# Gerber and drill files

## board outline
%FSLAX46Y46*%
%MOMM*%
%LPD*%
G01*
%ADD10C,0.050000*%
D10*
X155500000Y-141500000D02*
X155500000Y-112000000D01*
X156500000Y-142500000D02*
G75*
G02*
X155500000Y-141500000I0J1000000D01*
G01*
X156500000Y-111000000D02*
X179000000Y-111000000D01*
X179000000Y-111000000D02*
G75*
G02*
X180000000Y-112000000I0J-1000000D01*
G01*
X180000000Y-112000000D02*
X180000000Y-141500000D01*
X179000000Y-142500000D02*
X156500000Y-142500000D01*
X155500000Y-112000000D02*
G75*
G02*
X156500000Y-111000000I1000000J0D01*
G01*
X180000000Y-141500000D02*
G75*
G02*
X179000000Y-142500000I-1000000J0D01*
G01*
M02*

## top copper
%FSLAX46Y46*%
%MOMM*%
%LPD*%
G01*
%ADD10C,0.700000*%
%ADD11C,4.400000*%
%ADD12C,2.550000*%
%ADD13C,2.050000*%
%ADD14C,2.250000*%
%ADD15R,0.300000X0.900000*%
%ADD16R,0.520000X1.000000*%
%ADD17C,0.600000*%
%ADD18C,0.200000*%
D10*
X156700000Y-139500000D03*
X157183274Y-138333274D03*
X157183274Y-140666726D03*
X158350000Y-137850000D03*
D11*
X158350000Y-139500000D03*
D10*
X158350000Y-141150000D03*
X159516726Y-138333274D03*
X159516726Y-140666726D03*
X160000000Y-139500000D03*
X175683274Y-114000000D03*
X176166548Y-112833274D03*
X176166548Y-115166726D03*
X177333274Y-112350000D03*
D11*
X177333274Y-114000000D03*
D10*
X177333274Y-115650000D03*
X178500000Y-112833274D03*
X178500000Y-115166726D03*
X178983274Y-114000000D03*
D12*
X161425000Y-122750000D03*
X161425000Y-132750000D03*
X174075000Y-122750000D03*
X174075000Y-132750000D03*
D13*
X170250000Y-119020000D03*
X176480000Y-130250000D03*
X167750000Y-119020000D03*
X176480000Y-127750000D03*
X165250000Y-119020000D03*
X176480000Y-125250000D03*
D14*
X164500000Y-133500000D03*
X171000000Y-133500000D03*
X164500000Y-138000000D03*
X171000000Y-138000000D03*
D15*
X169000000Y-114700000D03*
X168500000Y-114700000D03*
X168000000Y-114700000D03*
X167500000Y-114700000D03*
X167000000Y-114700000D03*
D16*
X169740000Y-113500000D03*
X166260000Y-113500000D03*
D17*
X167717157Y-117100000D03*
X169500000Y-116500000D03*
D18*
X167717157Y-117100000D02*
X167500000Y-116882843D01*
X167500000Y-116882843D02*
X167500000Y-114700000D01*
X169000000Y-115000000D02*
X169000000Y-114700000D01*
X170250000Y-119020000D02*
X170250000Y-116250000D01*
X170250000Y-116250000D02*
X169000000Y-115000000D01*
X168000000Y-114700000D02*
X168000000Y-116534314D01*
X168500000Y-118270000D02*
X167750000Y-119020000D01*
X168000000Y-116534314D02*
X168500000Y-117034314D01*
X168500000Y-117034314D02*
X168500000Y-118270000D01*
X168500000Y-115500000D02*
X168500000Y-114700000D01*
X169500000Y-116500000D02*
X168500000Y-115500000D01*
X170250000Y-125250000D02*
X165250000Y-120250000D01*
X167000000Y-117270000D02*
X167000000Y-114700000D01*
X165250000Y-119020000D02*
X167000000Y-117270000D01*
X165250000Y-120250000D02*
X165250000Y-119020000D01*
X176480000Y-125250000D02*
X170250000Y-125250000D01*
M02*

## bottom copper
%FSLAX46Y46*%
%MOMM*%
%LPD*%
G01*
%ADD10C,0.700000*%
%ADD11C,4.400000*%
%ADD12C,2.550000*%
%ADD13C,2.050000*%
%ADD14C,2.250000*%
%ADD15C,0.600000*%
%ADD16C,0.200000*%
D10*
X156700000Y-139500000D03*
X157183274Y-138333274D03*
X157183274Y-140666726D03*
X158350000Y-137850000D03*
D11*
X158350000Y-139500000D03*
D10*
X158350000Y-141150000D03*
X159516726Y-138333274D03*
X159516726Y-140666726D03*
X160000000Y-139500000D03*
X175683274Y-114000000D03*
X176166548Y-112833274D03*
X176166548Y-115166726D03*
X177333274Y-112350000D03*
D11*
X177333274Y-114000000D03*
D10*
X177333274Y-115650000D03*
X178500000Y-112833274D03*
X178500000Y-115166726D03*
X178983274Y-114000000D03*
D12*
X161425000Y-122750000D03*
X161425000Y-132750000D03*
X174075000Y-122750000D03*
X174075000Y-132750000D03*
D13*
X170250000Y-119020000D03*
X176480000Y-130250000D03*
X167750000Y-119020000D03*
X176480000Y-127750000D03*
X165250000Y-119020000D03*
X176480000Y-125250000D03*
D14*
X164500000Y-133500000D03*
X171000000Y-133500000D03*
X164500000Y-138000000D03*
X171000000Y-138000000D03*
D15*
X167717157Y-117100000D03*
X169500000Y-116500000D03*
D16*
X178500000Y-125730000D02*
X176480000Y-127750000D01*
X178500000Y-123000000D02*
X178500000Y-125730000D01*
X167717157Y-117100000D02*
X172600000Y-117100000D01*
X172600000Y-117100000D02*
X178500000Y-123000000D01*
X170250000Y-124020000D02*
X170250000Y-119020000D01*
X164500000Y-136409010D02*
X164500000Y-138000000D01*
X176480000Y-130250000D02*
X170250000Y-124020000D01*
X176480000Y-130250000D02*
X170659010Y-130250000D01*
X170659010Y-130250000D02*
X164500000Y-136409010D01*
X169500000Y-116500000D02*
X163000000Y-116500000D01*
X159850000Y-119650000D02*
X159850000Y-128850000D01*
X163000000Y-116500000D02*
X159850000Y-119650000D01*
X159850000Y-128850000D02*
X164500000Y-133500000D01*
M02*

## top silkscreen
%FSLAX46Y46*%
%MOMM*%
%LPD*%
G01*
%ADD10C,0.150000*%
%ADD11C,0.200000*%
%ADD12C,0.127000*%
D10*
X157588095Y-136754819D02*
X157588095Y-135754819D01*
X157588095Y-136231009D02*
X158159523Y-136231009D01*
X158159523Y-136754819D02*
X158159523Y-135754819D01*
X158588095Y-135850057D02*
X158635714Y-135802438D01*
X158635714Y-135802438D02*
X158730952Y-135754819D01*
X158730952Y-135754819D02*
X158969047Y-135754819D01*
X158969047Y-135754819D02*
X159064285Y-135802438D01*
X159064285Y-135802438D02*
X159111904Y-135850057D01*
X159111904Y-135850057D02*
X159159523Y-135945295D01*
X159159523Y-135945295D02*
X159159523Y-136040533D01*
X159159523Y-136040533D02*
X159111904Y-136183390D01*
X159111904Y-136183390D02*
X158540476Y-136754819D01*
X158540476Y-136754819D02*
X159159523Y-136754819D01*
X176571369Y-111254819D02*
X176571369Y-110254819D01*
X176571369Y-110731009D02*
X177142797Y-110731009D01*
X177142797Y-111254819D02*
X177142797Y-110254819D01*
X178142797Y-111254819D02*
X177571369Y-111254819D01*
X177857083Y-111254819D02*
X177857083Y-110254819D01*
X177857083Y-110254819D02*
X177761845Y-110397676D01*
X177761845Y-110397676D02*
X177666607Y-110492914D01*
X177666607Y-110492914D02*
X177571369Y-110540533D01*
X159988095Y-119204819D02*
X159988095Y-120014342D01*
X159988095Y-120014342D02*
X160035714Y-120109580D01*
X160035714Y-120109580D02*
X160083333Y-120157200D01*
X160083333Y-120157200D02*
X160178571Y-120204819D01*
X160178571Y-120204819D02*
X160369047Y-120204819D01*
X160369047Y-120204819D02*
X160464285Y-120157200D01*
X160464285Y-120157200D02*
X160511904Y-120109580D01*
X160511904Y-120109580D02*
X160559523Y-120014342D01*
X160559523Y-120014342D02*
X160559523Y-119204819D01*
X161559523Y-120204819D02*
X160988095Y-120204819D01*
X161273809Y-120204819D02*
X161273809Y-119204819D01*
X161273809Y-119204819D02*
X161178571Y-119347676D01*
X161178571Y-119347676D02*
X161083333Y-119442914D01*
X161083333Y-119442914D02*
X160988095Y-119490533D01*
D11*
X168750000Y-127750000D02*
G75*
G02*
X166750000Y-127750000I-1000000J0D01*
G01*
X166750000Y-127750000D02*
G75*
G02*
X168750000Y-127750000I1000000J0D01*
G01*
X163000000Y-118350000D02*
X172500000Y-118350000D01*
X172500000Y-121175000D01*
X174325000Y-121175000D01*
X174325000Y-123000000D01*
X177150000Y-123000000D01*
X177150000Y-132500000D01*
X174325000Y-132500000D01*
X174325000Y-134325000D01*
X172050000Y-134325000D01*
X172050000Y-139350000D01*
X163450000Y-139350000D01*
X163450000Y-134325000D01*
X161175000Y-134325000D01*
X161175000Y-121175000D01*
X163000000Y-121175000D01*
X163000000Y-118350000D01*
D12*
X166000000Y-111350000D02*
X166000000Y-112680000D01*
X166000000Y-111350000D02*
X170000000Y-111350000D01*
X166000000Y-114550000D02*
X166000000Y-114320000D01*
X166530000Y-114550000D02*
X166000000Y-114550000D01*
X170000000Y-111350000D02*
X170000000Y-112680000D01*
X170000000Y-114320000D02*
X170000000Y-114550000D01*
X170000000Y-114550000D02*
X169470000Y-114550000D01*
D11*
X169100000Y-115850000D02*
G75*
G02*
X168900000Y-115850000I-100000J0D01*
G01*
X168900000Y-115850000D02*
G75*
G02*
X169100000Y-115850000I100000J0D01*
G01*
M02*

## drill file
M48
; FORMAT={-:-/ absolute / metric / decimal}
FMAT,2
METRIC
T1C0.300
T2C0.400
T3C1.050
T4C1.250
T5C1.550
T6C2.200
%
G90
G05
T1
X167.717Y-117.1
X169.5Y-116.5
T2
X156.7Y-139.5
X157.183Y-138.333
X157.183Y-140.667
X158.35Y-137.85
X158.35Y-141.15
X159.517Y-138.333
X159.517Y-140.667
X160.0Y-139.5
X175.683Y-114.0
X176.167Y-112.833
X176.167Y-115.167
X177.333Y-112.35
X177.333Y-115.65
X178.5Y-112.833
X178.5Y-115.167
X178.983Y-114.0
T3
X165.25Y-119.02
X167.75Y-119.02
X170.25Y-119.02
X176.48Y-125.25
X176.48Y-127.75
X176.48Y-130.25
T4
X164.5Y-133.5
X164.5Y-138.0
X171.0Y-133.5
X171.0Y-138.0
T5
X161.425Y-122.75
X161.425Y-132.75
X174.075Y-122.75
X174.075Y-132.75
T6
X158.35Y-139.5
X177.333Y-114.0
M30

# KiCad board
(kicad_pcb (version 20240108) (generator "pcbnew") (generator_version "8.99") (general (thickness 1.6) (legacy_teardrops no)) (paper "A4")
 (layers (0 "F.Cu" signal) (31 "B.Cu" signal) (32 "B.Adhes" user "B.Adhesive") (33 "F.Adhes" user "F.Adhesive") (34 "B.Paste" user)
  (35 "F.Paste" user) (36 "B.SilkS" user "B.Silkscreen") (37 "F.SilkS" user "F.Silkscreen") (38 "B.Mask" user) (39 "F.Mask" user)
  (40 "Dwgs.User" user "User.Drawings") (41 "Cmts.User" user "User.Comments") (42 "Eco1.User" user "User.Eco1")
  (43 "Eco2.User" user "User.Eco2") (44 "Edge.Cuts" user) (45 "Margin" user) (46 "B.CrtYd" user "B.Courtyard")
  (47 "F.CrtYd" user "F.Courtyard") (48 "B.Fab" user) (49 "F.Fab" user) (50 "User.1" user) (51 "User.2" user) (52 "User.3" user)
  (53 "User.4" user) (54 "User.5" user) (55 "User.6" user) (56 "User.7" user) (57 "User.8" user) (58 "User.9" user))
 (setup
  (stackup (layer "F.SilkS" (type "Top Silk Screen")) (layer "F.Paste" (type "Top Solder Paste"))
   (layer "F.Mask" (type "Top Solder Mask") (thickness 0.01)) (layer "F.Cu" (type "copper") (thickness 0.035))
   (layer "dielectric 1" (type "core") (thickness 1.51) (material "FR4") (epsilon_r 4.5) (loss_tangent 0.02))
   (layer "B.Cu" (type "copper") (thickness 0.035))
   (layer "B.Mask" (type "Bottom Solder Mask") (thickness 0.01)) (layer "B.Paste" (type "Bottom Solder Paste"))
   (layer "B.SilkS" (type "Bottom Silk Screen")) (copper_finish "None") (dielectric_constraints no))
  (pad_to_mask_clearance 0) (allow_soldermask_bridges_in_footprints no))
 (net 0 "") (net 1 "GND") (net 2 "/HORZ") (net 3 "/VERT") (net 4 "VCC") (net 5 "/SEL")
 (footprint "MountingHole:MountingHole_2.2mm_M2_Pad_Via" (layer "F.Cu") (at 158.35 139.5)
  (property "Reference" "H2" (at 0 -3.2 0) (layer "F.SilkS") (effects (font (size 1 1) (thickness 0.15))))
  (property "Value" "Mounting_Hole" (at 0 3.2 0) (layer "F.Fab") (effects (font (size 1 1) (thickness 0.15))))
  (pad "1" thru_hole circle (at -1.65 0) (size 0.7 0.7) (drill 0.4) (layers "*.Cu" "*.Mask") (remove_unused_layers no) (zone_connect 2))
  (pad "1" thru_hole circle (at -1.166726 -1.166726) (size 0.7 0.7) (drill 0.4) (layers "*.Cu" "*.Mask") (remove_unused_layers no)
   (zone_connect 2))
  (pad "1" thru_hole circle (at -1.166726 1.166726) (size 0.7 0.7) (drill 0.4) (layers "*.Cu" "*.Mask") (remove_unused_layers no)
   (zone_connect 2))
  (pad "1" thru_hole circle (at 0 -1.65) (size 0.7 0.7) (drill 0.4) (layers "*.Cu" "*.Mask") (remove_unused_layers no) (zone_connect 2))
  (pad "1" thru_hole circle (at 0 0) (size 4.4 4.4) (drill 2.2) (layers "*.Cu" "*.Mask") (remove_unused_layers no))
  (pad "1" thru_hole circle (at 0 1.65) (size 0.7 0.7) (drill 0.4) (layers "*.Cu" "*.Mask") (remove_unused_layers no) (zone_connect 2))
  (pad "1" thru_hole circle (at 1.166726 -1.166726) (size 0.7 0.7) (drill 0.4) (layers "*.Cu" "*.Mask") (remove_unused_layers no)
   (zone_connect 2))
  (pad "1" thru_hole circle (at 1.166726 1.166726) (size 0.7 0.7) (drill 0.4) (layers "*.Cu" "*.Mask") (remove_unused_layers no)
   (zone_connect 2))
  (pad "1" thru_hole circle (at 1.65 0) (size 0.7 0.7) (drill 0.4) (layers "*.Cu" "*.Mask") (remove_unused_layers no) (zone_connect 2)))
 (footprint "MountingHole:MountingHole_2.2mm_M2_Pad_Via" (layer "F.Cu") (at 177.333274 114)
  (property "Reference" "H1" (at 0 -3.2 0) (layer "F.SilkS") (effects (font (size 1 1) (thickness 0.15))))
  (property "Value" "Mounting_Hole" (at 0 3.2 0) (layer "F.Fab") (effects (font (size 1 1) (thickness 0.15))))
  (pad "1" thru_hole circle (at -1.65 0) (size 0.7 0.7) (drill 0.4) (layers "*.Cu" "*.Mask") (remove_unused_layers no) (zone_connect 2))
  (pad "1" thru_hole circle (at -1.166726 -1.166726) (size 0.7 0.7) (drill 0.4) (layers "*.Cu" "*.Mask") (remove_unused_layers no)
   (zone_connect 2))
  (pad "1" thru_hole circle (at -1.166726 1.166726) (size 0.7 0.7) (drill 0.4) (layers "*.Cu" "*.Mask") (remove_unused_layers no)
   (zone_connect 2))
  (pad "1" thru_hole circle (at 0 -1.65) (size 0.7 0.7) (drill 0.4) (layers "*.Cu" "*.Mask") (remove_unused_layers no) (zone_connect 2))
  (pad "1" thru_hole circle (at 0 0) (size 4.4 4.4) (drill 2.2) (layers "*.Cu" "*.Mask") (remove_unused_layers no))
  (pad "1" thru_hole circle (at 0 1.65) (size 0.7 0.7) (drill 0.4) (layers "*.Cu" "*.Mask") (remove_unused_layers no) (zone_connect 2))
  (pad "1" thru_hole circle (at 1.166726 -1.166726) (size 0.7 0.7) (drill 0.4) (layers "*.Cu" "*.Mask") (remove_unused_layers no)
   (zone_connect 2))
  (pad "1" thru_hole circle (at 1.166726 1.166726) (size 0.7 0.7) (drill 0.4) (layers "*.Cu" "*.Mask") (remove_unused_layers no)
   (zone_connect 2))
  (pad "1" thru_hole circle (at 1.65 0) (size 0.7 0.7) (drill 0.4) (layers "*.Cu" "*.Mask") (remove_unused_layers no) (zone_connect 2)))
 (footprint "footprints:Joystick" (layer "F.Cu") (at 167.75 127.75)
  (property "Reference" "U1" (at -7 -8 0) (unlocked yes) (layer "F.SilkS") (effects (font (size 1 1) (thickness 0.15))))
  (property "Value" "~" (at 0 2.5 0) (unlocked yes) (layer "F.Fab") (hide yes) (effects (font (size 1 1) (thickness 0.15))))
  (fp_circle (center 0 0) (end 1 0) (stroke (width 0.2) (type default)) (fill none) (layer "F.SilkS"))
  (fp_poly
   (pts (xy -4.75 -9.4) (xy 4.75 -9.4) (xy 4.75 -6.575) (xy 6.575 -6.575) (xy 6.575 -4.75) (xy 9.4 -4.75) (xy 9.4 4.75) (xy 6.575 4.75)
    (xy 6.575 6.575) (xy 4.3 6.575) (xy 4.3 11.6) (xy -4.3 11.6) (xy -4.3 6.575) (xy -6.575 6.575) (xy -6.575 -6.575) (xy -4.75 -6.575))
   (stroke (width 0.2) (type solid)) (fill none) (layer "F.SilkS"))
  (pad "" thru_hole circle (at -6.325 -5) (size 2.55 2.55) (drill 1.55) (layers "*.Cu" "*.Mask") (remove_unused_layers no)
   (solder_mask_margin 0.1))
  (pad "" thru_hole circle (at -6.325 5) (size 2.55 2.55) (drill 1.55) (layers "*.Cu" "*.Mask") (remove_unused_layers no)
   (solder_mask_margin 0.1))
  (pad "" thru_hole circle (at 6.325 -5) (size 2.55 2.55) (drill 1.55) (layers "*.Cu" "*.Mask") (remove_unused_layers no)
   (solder_mask_margin 0.1))
  (pad "" thru_hole circle (at 6.325 5) (size 2.55 2.55) (drill 1.55) (layers "*.Cu" "*.Mask") (remove_unused_layers no)
   (solder_mask_margin 0.1))
  (pad "1" thru_hole circle (at 2.5 -8.73) (size 2.05 2.05) (drill 1.05) (layers "*.Cu" "*.Mask") (remove_unused_layers no) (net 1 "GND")
   (solder_mask_margin 0.1))
  (pad "1'" thru_hole circle (at 8.73 2.5) (size 2.05 2.05) (drill 1.05) (layers "*.Cu" "*.Mask") (remove_unused_layers no) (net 1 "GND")
   (solder_mask_margin 0.1))
  (pad "2" thru_hole circle (at 0 -8.73) (size 2.05 2.05) (drill 1.05) (layers "*.Cu" "*.Mask") (remove_unused_layers no) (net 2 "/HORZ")
   (solder_mask_margin 0.1))
  (pad "2'" thru_hole circle (at 8.73 0) (size 2.05 2.05) (drill 1.05) (layers "*.Cu" "*.Mask") (remove_unused_layers no) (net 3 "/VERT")
   (solder_mask_margin 0.1))
  (pad "3" thru_hole circle (at -2.5 -8.73) (size 2.05 2.05) (drill 1.05) (layers "*.Cu" "*.Mask") (remove_unused_layers no) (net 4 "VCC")
   (solder_mask_margin 0.1))
  (pad "3'" thru_hole circle (at 8.73 -2.5) (size 2.05 2.05) (drill 1.05) (layers "*.Cu" "*.Mask") (remove_unused_layers no) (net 4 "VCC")
   (solder_mask_margin 0.1))
  (pad "a" thru_hole circle (at -3.25 5.75) (size 2.25 2.25) (drill 1.25) (layers "*.Cu" "*.Mask") (remove_unused_layers no) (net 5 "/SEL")
   (solder_mask_margin 0.1))
  (pad "b" thru_hole circle (at 3.25 5.75) (size 2.25 2.25) (drill 1.25) (layers "*.Cu" "*.Mask") (remove_unused_layers no)
   (solder_mask_margin 0.1))
  (pad "c" thru_hole circle (at -3.25 10.25) (size 2.25 2.25) (drill 1.25) (layers "*.Cu" "*.Mask") (remove_unused_layers no) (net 1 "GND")
   (solder_mask_margin 0.1))
  (pad "d" thru_hole circle (at 3.25 10.25) (size 2.25 2.25) (drill 1.25) (layers "*.Cu" "*.Mask") (remove_unused_layers no)
   (solder_mask_margin 0.1)))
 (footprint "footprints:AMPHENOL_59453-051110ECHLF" (layer "F.Cu") (at 168 113.5 180)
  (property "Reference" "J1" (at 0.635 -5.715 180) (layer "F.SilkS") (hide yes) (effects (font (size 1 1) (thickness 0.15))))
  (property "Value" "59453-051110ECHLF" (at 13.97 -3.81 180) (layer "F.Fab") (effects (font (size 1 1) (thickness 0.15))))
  (fp_line (start 2 2.15) (end 2 0.82) (stroke (width 0.127) (type solid)) (layer "F.SilkS"))
  (fp_line (start 2 2.15) (end -2 2.15) (stroke (width 0.127) (type solid)) (layer "F.SilkS"))
  (fp_line (start 2 -1.05) (end 2 -0.82) (stroke (width 0.127) (type solid)) (layer "F.SilkS"))
  (fp_line (start 1.47 -1.05) (end 2 -1.05) (stroke (width 0.127) (type solid)) (layer "F.SilkS"))
  (fp_line (start -2 2.15) (end -2 0.82) (stroke (width 0.127) (type solid)) (layer "F.SilkS"))
  (fp_line (start -2 -0.82) (end -2 -1.05) (stroke (width 0.127) (type solid)) (layer "F.SilkS"))
  (fp_line (start -2 -1.05) (end -1.47 -1.05) (stroke (width 0.127) (type solid)) (layer "F.SilkS"))
  (fp_circle (center -1 -2.35) (end -0.9 -2.35) (stroke (width 0.2) (type solid)) (fill none) (layer "F.SilkS"))
  (pad "1" smd rect (at -1 -1.2 180) (size 0.3 0.9) (layers "F.Cu" "F.Paste" "F.Mask") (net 1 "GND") (solder_mask_margin 0.102))
  (pad "2" smd rect (at -0.5 -1.2 180) (size 0.3 0.9) (layers "F.Cu" "F.Paste" "F.Mask") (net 5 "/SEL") (solder_mask_margin 0.102))
  (pad "3" smd rect (at 0 -1.2 180) (size 0.3 0.9) (layers "F.Cu" "F.Paste" "F.Mask") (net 2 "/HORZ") (solder_mask_margin 0.102))
  (pad "4" smd rect (at 0.5 -1.2 180) (size 0.3 0.9) (layers "F.Cu" "F.Paste" "F.Mask") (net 3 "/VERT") (solder_mask_margin 0.102))
  (pad "5" smd rect (at 1 -1.2 180) (size 0.3 0.9) (layers "F.Cu" "F.Paste" "F.Mask") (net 4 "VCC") (solder_mask_margin 0.102))
  (pad "S1" smd rect (at -1.74 0 180) (size 0.52 1) (layers "F.Cu" "F.Paste" "F.Mask") (solder_mask_margin 0.102))
  (pad "S2" smd rect (at 1.74 0 180) (size 0.52 1) (layers "F.Cu" "F.Paste" "F.Mask") (solder_mask_margin 0.102)))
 (gr_line (start 155.5 141.5) (end 155.5 112) (stroke (width 0.05) (type default)) (layer "Edge.Cuts"))
 (gr_arc (start 156.5 142.5) (mid 155.792893 142.207107) (end 155.5 141.5) (stroke (width 0.05) (type default)) (layer "Edge.Cuts"))
 (gr_line (start 156.5 111) (end 179 111) (stroke (width 0.05) (type default)) (layer "Edge.Cuts"))
 (gr_arc (start 179 111) (mid 179.707107 111.292893) (end 180 112) (stroke (width 0.05) (type default)) (layer "Edge.Cuts"))
 (gr_line (start 180 112) (end 180 141.5) (stroke (width 0.05) (type default)) (layer "Edge.Cuts"))
 (gr_line (start 179 142.5) (end 156.5 142.5) (stroke (width 0.05) (type default)) (layer "Edge.Cuts"))
 (gr_arc (start 155.5 112) (mid 155.792893 111.292893) (end 156.5 111) (stroke (width 0.05) (type default)) (layer "Edge.Cuts"))
 (gr_arc (start 180 141.5) (mid 179.707107 142.207107) (end 179 142.5) (stroke (width 0.05) (type default)) (layer "Edge.Cuts"))
 (segment (start 167.717157 117.1) (end 167.5 116.882843) (width 0.2) (layer "F.Cu") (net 3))
 (segment (start 167.5 116.882843) (end 167.5 114.7) (width 0.2) (layer "F.Cu") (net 3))
 (via (at 167.717157 117.1) (size 0.6) (drill 0.3) (layers "F.Cu" "B.Cu") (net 3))
 (segment (start 178.5 125.73) (end 176.48 127.75) (width 0.2) (layer "B.Cu") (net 3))
 (segment (start 178.5 123) (end 178.5 125.73) (width 0.2) (layer "B.Cu") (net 3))
 (segment (start 167.717157 117.1) (end 172.6 117.1) (width 0.2) (layer "B.Cu") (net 3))
 (segment (start 172.6 117.1) (end 178.5 123) (width 0.2) (layer "B.Cu") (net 3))
 (segment (start 169 115) (end 169 114.7) (width 0.2) (layer "F.Cu") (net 1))
 (segment (start 170.25 119.02) (end 170.25 116.25) (width 0.2) (layer "F.Cu") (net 1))
 (segment (start 170.25 116.25) (end 169 115) (width 0.2) (layer "F.Cu") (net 1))
 (segment (start 170.25 124.02) (end 170.25 119.02) (width 0.2) (layer "B.Cu") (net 1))
 (segment (start 164.5 136.40901) (end 164.5 138) (width 0.2) (layer "B.Cu") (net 1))
 (segment (start 176.48 130.25) (end 170.25 124.02) (width 0.2) (layer "B.Cu") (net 1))
 (segment (start 176.48 130.25) (end 170.65901 130.25) (width 0.2) (layer "B.Cu") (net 1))
 (segment (start 170.65901 130.25) (end 164.5 136.40901) (width 0.2) (layer "B.Cu") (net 1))
 (segment (start 168 114.7) (end 168 116.534314) (width 0.2) (layer "F.Cu") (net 2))
 (segment (start 168.5 118.27) (end 167.75 119.02) (width 0.2) (layer "F.Cu") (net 2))
 (segment (start 168 116.534314) (end 168.5 117.034314) (width 0.2) (layer "F.Cu") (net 2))
 (segment (start 168.5 117.034314) (end 168.5 118.27) (width 0.2) (layer "F.Cu") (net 2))
 (segment (start 168.5 115.5) (end 168.5 114.7) (width 0.2) (layer "F.Cu") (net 5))
 (segment (start 169.5 116.5) (end 168.5 115.5) (width 0.2) (layer "F.Cu") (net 5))
 (via (at 169.5 116.5) (size 0.6) (drill 0.3) (layers "F.Cu" "B.Cu") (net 5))
 (segment (start 169.5 116.5) (end 163 116.5) (width 0.2) (layer "B.Cu") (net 5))
 (segment (start 159.85 119.65) (end 159.85 128.85) (width 0.2) (layer "B.Cu") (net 5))
 (segment (start 163 116.5) (end 159.85 119.65) (width 0.2) (layer "B.Cu") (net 5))
 (segment (start 159.85 128.85) (end 164.5 133.5) (width 0.2) (layer "B.Cu") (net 5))
 (segment (start 170.25 125.25) (end 165.25 120.25) (width 0.2) (layer "F.Cu") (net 4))
 (segment (start 167 117.27) (end 167 114.7) (width 0.2) (layer "F.Cu") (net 4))
 (segment (start 165.25 119.02) (end 167 117.27) (width 0.2) (layer "F.Cu") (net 4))
 (segment (start 165.25 120.25) (end 165.25 119.02) (width 0.2) (layer "F.Cu") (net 4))
 (segment (start 176.48 125.25) (end 170.25 125.25) (width 0.2) (layer "F.Cu") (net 4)))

